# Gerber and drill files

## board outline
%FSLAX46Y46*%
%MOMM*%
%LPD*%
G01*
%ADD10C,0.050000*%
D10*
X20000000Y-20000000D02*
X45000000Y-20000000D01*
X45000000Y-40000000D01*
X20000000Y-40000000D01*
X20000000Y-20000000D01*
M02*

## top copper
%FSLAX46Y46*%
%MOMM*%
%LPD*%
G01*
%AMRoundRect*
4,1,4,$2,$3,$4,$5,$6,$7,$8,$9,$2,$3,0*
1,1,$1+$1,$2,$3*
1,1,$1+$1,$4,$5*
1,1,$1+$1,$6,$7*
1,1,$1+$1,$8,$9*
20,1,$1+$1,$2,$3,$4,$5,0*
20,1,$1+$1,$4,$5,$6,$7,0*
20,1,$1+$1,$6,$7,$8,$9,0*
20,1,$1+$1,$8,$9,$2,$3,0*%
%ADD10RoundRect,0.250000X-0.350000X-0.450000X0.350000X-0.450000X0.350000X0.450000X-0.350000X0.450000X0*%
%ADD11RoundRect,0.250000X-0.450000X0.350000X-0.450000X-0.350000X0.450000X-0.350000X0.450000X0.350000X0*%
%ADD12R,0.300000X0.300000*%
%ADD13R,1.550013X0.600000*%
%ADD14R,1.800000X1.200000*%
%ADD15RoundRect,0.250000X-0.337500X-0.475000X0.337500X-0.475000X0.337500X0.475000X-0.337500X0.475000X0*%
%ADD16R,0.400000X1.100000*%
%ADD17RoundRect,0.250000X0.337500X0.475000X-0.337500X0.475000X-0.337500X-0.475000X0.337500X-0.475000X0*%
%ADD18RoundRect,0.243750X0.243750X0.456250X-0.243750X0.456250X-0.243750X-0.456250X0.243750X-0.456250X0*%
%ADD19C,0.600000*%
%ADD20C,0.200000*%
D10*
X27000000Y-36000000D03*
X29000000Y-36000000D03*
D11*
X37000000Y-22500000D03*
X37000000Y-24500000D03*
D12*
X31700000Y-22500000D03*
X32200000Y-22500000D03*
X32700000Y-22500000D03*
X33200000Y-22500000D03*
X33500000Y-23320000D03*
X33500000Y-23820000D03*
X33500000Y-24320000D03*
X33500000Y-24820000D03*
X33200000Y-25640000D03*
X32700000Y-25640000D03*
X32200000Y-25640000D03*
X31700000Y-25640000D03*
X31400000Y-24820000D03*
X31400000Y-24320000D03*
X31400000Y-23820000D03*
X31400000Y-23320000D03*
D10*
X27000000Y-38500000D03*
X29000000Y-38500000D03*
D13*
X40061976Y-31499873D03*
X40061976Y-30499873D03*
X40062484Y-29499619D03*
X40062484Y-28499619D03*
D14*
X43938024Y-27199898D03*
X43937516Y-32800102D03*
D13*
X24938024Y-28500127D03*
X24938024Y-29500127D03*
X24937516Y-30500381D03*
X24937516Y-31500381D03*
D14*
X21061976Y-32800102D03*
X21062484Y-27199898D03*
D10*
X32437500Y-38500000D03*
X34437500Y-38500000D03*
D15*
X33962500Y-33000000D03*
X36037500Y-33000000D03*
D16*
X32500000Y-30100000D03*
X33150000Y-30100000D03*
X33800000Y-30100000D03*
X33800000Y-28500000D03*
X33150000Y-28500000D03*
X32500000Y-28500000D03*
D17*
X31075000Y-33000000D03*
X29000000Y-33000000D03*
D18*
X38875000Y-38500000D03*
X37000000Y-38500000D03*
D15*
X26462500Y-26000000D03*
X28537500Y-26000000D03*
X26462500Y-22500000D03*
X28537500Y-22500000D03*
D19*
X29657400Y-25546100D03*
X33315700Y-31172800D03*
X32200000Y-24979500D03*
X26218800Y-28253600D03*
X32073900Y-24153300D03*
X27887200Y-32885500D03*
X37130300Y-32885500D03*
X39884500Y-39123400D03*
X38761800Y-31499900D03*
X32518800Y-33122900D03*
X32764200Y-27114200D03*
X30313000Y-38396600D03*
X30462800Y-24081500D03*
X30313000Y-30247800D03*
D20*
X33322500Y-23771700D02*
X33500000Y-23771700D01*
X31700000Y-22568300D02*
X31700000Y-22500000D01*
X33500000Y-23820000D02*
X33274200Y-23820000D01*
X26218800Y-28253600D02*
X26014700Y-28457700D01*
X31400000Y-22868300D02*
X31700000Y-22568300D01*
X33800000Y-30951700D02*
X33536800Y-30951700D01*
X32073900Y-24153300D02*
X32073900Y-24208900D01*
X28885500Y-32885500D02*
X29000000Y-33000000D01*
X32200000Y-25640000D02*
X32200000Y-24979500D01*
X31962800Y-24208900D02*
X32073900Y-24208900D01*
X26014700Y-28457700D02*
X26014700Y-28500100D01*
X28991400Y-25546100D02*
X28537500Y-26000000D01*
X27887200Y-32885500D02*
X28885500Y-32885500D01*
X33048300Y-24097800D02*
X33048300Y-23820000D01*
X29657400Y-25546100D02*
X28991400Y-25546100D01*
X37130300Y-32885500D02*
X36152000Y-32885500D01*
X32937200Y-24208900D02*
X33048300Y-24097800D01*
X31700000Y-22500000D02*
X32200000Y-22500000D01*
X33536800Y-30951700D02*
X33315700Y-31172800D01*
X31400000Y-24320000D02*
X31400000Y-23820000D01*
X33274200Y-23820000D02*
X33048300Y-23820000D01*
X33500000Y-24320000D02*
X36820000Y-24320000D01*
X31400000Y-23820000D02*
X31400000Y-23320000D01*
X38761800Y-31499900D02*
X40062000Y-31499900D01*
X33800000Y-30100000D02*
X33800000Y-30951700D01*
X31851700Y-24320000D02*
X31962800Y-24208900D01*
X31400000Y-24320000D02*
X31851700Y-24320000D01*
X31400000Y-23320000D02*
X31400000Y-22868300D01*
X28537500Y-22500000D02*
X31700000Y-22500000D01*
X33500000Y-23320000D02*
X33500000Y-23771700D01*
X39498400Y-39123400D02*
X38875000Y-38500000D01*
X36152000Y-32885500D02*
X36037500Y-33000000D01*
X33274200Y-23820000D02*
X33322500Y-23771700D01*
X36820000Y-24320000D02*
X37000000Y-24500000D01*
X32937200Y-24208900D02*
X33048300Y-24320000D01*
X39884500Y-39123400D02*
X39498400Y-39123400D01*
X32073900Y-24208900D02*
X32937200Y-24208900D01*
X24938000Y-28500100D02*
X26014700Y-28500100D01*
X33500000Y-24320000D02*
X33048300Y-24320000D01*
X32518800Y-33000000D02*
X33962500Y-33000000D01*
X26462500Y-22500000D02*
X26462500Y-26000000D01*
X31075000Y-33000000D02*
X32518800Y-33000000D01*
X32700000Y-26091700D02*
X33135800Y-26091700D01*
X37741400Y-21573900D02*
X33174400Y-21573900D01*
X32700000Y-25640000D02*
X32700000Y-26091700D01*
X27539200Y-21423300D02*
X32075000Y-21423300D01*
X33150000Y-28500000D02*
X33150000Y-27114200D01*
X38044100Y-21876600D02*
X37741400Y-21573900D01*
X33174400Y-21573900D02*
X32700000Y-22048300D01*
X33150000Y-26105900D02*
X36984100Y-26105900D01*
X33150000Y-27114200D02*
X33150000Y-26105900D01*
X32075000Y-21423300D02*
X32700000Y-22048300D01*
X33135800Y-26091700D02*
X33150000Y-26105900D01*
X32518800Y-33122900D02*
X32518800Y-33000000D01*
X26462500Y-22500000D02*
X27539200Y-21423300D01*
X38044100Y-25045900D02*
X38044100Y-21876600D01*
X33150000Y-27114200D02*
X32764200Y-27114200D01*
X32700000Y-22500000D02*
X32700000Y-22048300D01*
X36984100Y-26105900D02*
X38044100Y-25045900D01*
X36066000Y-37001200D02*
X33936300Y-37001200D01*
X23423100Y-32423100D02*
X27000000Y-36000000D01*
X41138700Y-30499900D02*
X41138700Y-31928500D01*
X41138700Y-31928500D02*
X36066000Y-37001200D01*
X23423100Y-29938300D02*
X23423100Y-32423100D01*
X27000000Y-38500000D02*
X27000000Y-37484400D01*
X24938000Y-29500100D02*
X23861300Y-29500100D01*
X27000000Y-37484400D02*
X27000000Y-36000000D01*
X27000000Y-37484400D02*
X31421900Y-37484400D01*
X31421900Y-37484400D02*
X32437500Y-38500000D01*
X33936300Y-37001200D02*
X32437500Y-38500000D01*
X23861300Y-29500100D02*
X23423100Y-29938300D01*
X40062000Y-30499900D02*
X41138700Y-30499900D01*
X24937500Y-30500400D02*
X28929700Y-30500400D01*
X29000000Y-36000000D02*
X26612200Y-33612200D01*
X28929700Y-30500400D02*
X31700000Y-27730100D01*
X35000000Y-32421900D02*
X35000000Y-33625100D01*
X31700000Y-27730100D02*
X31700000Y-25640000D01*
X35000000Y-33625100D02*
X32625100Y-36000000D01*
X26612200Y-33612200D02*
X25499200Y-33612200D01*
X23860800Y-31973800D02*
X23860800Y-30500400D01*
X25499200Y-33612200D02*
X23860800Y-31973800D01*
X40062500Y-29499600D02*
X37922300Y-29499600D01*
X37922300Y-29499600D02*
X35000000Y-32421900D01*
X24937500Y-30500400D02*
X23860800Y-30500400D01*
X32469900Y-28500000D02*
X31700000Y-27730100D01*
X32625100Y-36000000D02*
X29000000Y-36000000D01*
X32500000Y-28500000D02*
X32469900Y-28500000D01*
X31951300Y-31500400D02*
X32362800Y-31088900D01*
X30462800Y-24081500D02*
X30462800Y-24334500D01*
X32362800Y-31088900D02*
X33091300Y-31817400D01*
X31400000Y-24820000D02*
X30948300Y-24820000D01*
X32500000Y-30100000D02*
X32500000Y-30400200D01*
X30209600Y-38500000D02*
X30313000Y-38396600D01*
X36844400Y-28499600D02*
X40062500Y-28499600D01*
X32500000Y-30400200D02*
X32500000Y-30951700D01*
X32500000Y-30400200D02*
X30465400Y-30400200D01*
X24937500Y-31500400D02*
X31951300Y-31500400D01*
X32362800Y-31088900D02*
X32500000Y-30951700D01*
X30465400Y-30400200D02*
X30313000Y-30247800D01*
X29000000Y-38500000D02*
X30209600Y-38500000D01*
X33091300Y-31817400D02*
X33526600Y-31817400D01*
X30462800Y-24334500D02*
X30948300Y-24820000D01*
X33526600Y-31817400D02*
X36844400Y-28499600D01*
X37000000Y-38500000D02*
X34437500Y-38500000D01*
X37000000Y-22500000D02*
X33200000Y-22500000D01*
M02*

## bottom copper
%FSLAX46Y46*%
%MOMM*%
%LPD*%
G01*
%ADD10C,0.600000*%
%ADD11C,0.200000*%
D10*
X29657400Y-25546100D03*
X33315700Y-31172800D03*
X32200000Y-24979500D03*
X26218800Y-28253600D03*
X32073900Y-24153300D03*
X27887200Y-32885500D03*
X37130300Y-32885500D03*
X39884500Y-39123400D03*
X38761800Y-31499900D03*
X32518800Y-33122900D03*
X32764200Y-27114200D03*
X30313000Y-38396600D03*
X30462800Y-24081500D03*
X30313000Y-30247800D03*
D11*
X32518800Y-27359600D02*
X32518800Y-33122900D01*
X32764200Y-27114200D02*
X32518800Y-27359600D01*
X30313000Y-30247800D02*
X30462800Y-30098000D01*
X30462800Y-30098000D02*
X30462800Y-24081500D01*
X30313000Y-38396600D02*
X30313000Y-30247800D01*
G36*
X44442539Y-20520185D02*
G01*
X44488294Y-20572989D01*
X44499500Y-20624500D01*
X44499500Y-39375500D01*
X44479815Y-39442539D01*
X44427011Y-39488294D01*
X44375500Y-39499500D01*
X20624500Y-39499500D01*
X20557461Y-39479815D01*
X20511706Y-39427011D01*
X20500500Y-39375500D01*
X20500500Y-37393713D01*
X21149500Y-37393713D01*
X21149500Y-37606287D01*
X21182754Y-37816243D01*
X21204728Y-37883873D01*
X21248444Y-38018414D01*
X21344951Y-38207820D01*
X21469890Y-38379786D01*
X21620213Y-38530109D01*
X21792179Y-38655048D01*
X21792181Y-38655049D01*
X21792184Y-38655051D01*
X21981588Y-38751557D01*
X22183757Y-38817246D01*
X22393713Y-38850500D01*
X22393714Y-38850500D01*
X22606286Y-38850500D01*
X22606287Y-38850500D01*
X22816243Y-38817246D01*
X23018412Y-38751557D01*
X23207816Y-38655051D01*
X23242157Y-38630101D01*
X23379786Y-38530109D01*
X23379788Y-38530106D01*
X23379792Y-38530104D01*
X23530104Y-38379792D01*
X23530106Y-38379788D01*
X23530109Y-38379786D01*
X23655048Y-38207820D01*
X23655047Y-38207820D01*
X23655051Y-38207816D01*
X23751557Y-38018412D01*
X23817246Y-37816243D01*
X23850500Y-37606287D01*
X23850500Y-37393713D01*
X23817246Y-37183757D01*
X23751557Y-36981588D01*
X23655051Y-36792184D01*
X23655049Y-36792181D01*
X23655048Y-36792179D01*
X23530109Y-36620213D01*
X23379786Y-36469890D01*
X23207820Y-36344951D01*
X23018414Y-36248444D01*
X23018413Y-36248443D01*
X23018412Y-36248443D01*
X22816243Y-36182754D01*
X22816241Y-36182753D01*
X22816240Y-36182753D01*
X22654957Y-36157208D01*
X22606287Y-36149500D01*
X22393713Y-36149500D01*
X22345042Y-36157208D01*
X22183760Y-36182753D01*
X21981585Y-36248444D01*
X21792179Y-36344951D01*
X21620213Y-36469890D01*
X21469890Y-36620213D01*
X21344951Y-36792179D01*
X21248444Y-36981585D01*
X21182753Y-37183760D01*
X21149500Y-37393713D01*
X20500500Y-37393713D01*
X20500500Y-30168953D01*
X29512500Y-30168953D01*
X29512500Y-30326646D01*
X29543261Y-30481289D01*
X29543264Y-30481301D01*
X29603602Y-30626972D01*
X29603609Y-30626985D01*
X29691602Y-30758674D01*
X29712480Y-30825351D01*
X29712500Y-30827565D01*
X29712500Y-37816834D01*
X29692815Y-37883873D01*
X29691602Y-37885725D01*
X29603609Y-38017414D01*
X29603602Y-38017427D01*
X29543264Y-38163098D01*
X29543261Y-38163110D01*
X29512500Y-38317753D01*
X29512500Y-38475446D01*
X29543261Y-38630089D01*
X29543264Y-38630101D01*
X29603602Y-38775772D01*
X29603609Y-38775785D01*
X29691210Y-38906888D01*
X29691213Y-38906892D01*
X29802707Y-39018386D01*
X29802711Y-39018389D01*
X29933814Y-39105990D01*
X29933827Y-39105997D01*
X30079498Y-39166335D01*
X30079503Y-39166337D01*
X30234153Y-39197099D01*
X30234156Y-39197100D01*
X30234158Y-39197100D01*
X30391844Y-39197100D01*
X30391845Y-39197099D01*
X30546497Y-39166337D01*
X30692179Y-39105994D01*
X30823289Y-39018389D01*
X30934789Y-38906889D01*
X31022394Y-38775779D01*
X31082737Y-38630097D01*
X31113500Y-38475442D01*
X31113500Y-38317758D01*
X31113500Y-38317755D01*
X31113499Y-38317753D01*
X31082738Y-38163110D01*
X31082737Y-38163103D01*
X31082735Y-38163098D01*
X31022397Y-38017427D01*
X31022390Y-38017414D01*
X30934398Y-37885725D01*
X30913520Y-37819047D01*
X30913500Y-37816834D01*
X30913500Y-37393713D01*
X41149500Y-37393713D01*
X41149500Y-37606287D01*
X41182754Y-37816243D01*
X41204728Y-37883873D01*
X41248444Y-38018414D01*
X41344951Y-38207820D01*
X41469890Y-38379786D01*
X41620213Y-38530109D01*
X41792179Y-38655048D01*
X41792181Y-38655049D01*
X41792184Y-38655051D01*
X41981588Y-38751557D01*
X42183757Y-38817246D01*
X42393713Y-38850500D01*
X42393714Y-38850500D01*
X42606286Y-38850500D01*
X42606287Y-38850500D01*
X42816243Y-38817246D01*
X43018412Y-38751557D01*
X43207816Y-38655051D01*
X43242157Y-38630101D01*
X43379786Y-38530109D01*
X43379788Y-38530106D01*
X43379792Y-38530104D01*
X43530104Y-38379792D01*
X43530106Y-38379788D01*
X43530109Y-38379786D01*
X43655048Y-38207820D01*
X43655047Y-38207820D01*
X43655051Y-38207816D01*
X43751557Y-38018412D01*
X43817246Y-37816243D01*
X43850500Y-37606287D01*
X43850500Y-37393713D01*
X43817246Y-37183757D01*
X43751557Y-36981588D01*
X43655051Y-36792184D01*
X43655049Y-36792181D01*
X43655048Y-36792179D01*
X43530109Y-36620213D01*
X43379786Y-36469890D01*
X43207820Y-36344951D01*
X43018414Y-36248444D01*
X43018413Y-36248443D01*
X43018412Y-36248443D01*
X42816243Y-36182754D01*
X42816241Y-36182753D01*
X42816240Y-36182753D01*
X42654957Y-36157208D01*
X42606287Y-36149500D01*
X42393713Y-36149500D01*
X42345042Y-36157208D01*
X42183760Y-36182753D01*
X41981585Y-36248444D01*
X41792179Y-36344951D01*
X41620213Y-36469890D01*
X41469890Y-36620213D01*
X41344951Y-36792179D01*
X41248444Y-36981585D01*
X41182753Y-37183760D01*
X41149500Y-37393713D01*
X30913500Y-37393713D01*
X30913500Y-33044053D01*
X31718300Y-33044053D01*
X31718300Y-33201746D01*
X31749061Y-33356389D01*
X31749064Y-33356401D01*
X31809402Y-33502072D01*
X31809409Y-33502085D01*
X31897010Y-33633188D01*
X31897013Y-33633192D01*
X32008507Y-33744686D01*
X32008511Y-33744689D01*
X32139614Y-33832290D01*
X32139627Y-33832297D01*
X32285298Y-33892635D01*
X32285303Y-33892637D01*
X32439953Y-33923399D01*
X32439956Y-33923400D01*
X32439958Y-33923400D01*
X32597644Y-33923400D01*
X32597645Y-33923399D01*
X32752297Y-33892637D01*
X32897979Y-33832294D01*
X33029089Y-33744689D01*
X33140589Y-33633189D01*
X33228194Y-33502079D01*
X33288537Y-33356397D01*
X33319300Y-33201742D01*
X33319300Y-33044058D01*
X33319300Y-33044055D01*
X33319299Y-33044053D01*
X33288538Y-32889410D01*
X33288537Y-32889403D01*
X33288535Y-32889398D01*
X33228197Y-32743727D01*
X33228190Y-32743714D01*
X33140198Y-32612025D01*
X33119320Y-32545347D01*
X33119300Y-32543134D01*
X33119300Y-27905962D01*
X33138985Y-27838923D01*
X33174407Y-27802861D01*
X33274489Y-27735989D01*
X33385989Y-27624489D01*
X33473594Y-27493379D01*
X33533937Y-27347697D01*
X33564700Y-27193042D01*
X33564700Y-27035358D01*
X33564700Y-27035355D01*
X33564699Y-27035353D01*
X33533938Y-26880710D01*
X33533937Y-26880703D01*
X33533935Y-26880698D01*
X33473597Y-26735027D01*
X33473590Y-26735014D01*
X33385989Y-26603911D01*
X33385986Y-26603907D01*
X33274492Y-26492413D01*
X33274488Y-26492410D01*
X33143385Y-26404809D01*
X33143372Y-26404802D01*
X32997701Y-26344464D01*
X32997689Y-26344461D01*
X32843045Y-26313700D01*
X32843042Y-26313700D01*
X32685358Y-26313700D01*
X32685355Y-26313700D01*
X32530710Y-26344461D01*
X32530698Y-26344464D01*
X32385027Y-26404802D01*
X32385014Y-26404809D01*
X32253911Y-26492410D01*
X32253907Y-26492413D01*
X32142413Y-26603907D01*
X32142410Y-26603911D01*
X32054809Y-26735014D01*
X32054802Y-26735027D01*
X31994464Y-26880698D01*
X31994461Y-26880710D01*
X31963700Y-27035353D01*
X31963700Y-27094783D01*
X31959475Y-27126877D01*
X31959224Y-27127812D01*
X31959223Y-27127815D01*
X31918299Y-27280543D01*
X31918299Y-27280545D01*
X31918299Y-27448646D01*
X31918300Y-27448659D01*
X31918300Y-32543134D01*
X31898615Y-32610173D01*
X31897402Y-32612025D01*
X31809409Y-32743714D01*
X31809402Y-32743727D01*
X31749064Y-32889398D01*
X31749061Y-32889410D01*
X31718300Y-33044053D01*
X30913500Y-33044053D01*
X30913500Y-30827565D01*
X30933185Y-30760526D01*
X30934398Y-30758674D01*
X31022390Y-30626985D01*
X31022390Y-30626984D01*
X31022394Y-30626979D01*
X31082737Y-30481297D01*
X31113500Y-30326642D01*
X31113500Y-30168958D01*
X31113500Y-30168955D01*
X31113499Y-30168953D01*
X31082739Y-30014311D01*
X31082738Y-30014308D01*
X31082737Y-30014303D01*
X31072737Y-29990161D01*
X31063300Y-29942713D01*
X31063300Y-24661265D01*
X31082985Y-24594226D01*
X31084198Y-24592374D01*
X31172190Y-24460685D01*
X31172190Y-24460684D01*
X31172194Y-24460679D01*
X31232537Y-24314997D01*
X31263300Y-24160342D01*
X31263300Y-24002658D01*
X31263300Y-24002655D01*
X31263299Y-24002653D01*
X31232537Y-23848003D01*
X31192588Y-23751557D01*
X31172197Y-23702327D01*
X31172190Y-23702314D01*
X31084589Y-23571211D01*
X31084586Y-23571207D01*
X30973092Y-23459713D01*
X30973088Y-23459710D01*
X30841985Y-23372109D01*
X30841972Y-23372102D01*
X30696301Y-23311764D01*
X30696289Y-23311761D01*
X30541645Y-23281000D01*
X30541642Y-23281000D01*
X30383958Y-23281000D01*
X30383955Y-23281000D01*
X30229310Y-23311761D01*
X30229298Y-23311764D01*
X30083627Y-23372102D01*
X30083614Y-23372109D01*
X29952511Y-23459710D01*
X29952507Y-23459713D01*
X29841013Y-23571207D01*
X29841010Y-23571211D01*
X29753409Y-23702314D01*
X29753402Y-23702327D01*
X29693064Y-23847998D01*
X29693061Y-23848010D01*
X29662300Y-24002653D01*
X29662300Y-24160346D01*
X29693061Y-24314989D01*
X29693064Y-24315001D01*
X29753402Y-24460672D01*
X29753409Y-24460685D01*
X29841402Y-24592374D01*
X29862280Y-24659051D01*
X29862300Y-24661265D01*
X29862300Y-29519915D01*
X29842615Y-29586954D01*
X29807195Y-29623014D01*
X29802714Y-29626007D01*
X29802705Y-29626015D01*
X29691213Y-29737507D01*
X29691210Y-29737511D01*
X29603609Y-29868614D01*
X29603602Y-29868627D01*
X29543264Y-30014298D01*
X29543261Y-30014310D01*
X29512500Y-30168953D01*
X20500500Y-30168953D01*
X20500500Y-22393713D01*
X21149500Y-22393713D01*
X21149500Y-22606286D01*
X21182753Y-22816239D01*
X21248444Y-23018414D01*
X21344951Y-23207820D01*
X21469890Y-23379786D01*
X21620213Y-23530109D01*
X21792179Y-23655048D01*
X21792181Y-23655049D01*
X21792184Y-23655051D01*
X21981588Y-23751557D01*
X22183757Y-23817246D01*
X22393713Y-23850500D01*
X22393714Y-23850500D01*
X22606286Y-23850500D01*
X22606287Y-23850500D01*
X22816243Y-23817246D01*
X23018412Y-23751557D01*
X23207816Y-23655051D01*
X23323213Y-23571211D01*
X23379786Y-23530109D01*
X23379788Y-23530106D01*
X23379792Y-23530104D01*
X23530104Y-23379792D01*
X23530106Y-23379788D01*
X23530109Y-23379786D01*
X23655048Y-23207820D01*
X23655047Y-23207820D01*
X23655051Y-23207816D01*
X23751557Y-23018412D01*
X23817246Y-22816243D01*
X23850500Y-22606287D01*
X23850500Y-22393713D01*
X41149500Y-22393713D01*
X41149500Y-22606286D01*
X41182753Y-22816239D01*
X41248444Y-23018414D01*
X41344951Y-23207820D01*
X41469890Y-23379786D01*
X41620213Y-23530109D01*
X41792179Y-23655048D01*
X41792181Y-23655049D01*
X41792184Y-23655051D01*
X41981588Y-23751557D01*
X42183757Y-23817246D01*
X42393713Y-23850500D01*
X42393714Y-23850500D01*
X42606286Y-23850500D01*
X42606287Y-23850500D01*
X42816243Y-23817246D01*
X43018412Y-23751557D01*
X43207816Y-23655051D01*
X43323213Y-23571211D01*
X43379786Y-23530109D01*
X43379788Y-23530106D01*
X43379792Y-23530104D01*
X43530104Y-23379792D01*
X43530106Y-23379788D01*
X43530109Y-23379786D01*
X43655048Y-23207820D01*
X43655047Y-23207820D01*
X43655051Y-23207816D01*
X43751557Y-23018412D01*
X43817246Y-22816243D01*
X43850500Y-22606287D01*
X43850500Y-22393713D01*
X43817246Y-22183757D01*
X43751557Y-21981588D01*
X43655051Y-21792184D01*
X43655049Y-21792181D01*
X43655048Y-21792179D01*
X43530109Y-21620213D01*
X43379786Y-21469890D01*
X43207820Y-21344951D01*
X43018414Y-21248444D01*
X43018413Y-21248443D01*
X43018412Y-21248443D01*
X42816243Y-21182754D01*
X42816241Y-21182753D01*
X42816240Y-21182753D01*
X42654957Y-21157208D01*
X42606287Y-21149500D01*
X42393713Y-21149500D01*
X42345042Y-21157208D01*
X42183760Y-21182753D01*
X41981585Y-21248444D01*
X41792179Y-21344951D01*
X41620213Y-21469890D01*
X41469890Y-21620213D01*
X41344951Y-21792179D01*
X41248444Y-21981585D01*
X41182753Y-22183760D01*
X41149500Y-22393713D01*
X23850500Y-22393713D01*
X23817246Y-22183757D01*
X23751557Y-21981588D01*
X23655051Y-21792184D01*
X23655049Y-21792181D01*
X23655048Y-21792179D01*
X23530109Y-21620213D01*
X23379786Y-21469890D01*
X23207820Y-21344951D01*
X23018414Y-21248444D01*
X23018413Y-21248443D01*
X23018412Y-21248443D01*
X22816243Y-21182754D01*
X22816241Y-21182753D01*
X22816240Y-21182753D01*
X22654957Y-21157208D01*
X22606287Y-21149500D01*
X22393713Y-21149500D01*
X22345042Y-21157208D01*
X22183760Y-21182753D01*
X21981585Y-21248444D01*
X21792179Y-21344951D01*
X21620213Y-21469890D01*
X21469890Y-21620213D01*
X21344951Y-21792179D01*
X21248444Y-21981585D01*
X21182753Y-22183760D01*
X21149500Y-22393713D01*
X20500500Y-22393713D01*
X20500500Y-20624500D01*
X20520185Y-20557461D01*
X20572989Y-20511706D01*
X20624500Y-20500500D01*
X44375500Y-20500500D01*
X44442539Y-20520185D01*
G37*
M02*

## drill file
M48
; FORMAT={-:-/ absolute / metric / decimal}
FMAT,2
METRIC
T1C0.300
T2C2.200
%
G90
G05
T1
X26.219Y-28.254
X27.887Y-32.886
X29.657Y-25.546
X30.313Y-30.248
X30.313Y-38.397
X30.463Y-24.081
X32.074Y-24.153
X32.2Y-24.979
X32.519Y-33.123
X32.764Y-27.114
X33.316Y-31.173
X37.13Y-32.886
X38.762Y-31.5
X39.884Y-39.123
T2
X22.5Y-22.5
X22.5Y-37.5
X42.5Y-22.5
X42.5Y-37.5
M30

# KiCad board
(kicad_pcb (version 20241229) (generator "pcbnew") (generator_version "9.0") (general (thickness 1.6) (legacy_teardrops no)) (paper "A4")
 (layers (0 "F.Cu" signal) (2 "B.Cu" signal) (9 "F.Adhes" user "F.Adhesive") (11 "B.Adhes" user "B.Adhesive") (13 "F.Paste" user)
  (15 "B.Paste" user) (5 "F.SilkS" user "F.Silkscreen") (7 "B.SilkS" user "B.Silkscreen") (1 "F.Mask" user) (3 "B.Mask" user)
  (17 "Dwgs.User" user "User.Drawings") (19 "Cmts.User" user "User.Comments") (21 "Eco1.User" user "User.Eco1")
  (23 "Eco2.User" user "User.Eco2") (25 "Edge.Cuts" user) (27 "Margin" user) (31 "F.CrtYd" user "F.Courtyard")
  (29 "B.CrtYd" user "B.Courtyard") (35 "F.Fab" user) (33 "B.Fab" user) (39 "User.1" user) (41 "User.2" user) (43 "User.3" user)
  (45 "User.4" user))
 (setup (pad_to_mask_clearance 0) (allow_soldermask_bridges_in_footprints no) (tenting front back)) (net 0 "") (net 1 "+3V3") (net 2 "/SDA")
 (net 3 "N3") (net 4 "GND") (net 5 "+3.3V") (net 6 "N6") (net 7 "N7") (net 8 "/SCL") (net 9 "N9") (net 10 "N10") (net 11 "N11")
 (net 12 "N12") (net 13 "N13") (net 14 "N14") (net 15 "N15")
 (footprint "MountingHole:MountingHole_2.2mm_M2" (layer "F.Cu") (at 22.5 22.5)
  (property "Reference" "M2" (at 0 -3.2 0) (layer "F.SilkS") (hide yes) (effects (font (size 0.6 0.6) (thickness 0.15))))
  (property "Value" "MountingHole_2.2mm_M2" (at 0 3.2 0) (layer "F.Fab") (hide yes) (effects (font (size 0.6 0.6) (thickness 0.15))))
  (pad "" np_thru_hole circle (at 0 0) (size 2.2 2.2) (drill 2.2) (layers "*.Cu" "*.Mask")))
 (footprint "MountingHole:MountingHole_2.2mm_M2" (layer "F.Cu") (at 42.5 22.5)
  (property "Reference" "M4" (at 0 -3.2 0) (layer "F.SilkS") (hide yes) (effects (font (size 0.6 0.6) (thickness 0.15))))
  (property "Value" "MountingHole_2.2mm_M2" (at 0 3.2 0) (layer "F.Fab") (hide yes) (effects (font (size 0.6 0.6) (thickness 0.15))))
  (pad "" np_thru_hole circle (at 0 0) (size 2.2 2.2) (drill 2.2) (layers "*.Cu" "*.Mask")))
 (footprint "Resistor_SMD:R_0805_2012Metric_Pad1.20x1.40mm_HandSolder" (layer "F.Cu") (at 28 36)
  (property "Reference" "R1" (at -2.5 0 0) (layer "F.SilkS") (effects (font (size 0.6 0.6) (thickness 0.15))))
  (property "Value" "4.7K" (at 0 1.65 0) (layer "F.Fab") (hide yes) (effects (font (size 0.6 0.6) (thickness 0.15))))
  (pad "1" smd roundrect (at -1 0) (size 1.2 1.4) (layers "F.Cu" "F.Mask" "F.Paste") (roundrect_rratio 0.208333) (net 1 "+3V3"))
  (pad "2" smd roundrect (at 1 0) (size 1.2 1.4) (layers "F.Cu" "F.Mask" "F.Paste") (roundrect_rratio 0.208333) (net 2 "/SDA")))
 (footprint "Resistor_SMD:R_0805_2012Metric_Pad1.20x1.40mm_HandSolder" (layer "F.Cu") (at 37 23.5 -90)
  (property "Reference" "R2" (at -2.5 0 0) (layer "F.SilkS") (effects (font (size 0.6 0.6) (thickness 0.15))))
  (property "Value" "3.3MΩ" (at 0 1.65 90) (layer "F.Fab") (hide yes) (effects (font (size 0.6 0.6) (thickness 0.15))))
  (pad "1" smd roundrect (at -1 0 270) (size 1.2 1.4) (layers "F.Cu" "F.Mask" "F.Paste") (roundrect_rratio 0.208333) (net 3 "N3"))
  (pad "2" smd roundrect (at 1 0 270) (size 1.2 1.4) (layers "F.Cu" "F.Mask" "F.Paste") (roundrect_rratio 0.208333) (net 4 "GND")))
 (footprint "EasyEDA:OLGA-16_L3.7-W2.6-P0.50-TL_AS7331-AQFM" (layer "F.Cu") (at 32.45 24.07)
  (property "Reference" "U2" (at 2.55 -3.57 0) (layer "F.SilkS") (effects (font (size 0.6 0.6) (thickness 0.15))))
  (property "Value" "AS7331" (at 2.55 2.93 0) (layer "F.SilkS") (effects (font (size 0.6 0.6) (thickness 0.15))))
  (pad "1" smd rect (at -0.75 -1.57) (size 0.3 0.3) (layers "F.Cu" "F.Mask" "F.Paste") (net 4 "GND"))
  (pad "2" smd rect (at -0.25 -1.57) (size 0.3 0.3) (layers "F.Cu" "F.Mask" "F.Paste") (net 4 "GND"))
  (pad "3" smd rect (at 0.25 -1.57) (size 0.3 0.3) (layers "F.Cu" "F.Mask" "F.Paste") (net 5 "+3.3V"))
  (pad "4" smd rect (at 0.75 -1.57) (size 0.3 0.3) (layers "F.Cu" "F.Mask" "F.Paste") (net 3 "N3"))
  (pad "5" smd rect (at 1.05 -0.75) (size 0.3 0.3) (layers "F.Cu" "F.Mask" "F.Paste") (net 4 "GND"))
  (pad "6" smd rect (at 1.05 -0.25) (size 0.3 0.3) (layers "F.Cu" "F.Mask" "F.Paste") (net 4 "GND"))
  (pad "7" smd rect (at 1.05 0.25) (size 0.3 0.3) (layers "F.Cu" "F.Mask" "F.Paste") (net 4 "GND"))
  (pad "8" smd rect (at 1.05 0.75) (size 0.3 0.3) (layers "F.Cu" "F.Mask" "F.Paste") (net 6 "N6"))
  (pad "9" smd rect (at 0.75 1.57) (size 0.3 0.3) (layers "F.Cu" "F.Mask" "F.Paste") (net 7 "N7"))
  (pad "10" smd rect (at 0.25 1.57) (size 0.3 0.3) (layers "F.Cu" "F.Mask" "F.Paste") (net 5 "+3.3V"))
  (pad "11" smd rect (at -0.25 1.57) (size 0.3 0.3) (layers "F.Cu" "F.Mask" "F.Paste") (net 4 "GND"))
  (pad "12" smd rect (at -0.75 1.57) (size 0.3 0.3) (layers "F.Cu" "F.Mask" "F.Paste") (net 2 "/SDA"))
  (pad "13" smd rect (at -1.05 0.75) (size 0.3 0.3) (layers "F.Cu" "F.Mask" "F.Paste") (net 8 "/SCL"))
  (pad "14" smd rect (at -1.05 0.25) (size 0.3 0.3) (layers "F.Cu" "F.Mask" "F.Paste") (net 4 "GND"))
  (pad "15" smd rect (at -1.05 -0.25) (size 0.3 0.3) (layers "F.Cu" "F.Mask" "F.Paste") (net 4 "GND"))
  (pad "16" smd rect (at -1.05 -0.75) (size 0.3 0.3) (layers "F.Cu" "F.Mask" "F.Paste") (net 4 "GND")))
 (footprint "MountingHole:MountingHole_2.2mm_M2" (layer "F.Cu") (at 42.5 37.5)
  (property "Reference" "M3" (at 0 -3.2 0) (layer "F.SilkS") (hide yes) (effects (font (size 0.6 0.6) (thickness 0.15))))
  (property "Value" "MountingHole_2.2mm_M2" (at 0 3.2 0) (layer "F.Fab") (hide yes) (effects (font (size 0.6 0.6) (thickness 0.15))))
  (pad "" np_thru_hole circle (at 0 0) (size 2.2 2.2) (drill 2.2) (layers "*.Cu" "*.Mask")))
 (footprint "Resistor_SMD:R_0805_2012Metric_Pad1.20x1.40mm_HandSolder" (layer "F.Cu") (at 28 38.5)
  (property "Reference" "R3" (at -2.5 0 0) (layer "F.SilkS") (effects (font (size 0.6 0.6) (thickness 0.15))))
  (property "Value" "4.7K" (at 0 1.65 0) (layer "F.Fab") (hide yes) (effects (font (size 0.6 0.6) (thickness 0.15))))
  (pad "1" smd roundrect (at -1 0) (size 1.2 1.4) (layers "F.Cu" "F.Mask" "F.Paste") (roundrect_rratio 0.208333) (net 1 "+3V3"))
  (pad "2" smd roundrect (at 1 0) (size 1.2 1.4) (layers "F.Cu" "F.Mask" "F.Paste") (roundrect_rratio 0.208333) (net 8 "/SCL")))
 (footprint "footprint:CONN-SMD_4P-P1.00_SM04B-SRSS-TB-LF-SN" (layer "F.Cu") (at 42 30 90)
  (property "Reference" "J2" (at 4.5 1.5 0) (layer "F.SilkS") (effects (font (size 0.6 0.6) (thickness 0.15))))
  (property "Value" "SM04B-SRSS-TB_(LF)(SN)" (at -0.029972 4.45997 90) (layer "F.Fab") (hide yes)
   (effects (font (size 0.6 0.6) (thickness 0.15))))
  (pad "1" smd rect (at -1.499873 -1.938024 90) (size 0.6 1.550013) (layers "F.Cu" "F.Mask" "F.Paste") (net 4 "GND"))
  (pad "2" smd rect (at -0.499873 -1.938024 90) (size 0.6 1.550013) (layers "F.Cu" "F.Mask" "F.Paste") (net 1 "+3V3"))
  (pad "3" smd rect (at 0.500381 -1.937516 90) (size 0.6 1.550013) (layers "F.Cu" "F.Mask" "F.Paste") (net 2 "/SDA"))
  (pad "4" smd rect (at 1.500381 -1.937516 90) (size 0.6 1.550013) (layers "F.Cu" "F.Mask" "F.Paste") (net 8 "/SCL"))
  (pad "5" smd rect (at 2.800102 1.938024 90) (size 1.2 1.8) (layers "F.Cu" "F.Mask" "F.Paste") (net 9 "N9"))
  (pad "6" smd rect (at -2.800102 1.937516 90) (size 1.2 1.8) (layers "F.Cu" "F.Mask" "F.Paste") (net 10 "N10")))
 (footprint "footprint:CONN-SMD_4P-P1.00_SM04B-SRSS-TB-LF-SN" (layer "F.Cu") (at 23 30 -90)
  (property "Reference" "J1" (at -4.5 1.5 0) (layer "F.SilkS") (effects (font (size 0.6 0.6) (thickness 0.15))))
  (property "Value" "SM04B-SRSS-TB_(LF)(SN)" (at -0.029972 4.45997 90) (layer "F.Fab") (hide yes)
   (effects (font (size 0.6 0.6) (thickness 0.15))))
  (pad "1" smd rect (at -1.499873 -1.938024 270) (size 0.6 1.550013) (layers "F.Cu" "F.Mask" "F.Paste") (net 4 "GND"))
  (pad "2" smd rect (at -0.499873 -1.938024 270) (size 0.6 1.550013) (layers "F.Cu" "F.Mask" "F.Paste") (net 1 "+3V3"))
  (pad "3" smd rect (at 0.500381 -1.937516 270) (size 0.6 1.550013) (layers "F.Cu" "F.Mask" "F.Paste") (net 2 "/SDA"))
  (pad "4" smd rect (at 1.500381 -1.937516 270) (size 0.6 1.550013) (layers "F.Cu" "F.Mask" "F.Paste") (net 8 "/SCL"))
  (pad "5" smd rect (at 2.800102 1.938024 270) (size 1.2 1.8) (layers "F.Cu" "F.Mask" "F.Paste") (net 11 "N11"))
  (pad "6" smd rect (at -2.800102 1.937516 270) (size 1.2 1.8) (layers "F.Cu" "F.Mask" "F.Paste") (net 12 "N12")))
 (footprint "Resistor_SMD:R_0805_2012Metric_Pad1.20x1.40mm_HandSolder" (layer "F.Cu") (at 33.4375 38.5)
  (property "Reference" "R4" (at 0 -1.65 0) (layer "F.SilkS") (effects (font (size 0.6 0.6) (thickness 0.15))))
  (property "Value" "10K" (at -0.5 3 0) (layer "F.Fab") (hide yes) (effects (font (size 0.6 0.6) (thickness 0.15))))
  (pad "1" smd roundrect (at -1 0) (size 1.2 1.4) (layers "F.Cu" "F.Mask" "F.Paste") (roundrect_rratio 0.208333) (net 1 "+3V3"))
  (pad "2" smd roundrect (at 1 0) (size 1.2 1.4) (layers "F.Cu" "F.Mask" "F.Paste") (roundrect_rratio 0.208333) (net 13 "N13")))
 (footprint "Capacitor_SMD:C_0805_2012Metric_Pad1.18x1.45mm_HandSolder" (layer "F.Cu") (at 35 33)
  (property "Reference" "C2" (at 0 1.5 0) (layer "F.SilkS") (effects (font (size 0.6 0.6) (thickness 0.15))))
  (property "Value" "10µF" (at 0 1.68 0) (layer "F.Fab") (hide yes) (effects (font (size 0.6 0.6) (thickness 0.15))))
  (pad "1" smd roundrect (at -1.0375 0) (size 1.175 1.45) (layers "F.Cu" "F.Mask" "F.Paste") (roundrect_rratio 0.212766) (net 5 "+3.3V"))
  (pad "2" smd roundrect (at 1.0375 0) (size 1.175 1.45) (layers "F.Cu" "F.Mask" "F.Paste") (roundrect_rratio 0.212766) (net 4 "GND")))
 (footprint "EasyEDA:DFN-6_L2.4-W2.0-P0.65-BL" (layer "F.Cu") (at 33.15 29.3)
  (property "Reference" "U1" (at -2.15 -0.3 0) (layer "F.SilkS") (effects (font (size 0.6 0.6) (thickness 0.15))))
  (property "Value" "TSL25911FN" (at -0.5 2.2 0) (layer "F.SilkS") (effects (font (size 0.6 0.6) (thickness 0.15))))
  (pad "1" smd rect (at -0.65 0.8) (size 0.4 1.1) (layers "F.Cu" "F.Mask" "F.Paste") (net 8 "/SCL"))
  (pad "2" smd rect (at 0 0.8) (size 0.4 1.1) (layers "F.Cu" "F.Mask" "F.Paste") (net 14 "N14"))
  (pad "3" smd rect (at 0.65 0.8) (size 0.4 1.1) (layers "F.Cu" "F.Mask" "F.Paste") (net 4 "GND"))
  (pad "4" smd rect (at 0.65 -0.8) (size 0.4 1.1) (layers "F.Cu" "F.Mask" "F.Paste") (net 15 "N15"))
  (pad "5" smd rect (at 0 -0.8) (size 0.4 1.1) (layers "F.Cu" "F.Mask" "F.Paste") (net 5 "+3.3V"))
  (pad "6" smd rect (at -0.65 -0.8) (size 0.4 1.1) (layers "F.Cu" "F.Mask" "F.Paste") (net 2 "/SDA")))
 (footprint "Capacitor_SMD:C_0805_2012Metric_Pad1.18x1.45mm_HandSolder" (layer "F.Cu") (at 30.0375 33 180)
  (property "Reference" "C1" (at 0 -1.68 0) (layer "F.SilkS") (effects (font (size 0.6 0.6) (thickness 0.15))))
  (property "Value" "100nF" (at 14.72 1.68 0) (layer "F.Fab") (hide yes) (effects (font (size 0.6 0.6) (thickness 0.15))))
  (pad "1" smd roundrect (at -1.0375 0 180) (size 1.175 1.45) (layers "F.Cu" "F.Mask" "F.Paste") (roundrect_rratio 0.212766) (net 5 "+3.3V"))
  (pad "2" smd roundrect (at 1.0375 0 180) (size 1.175 1.45) (layers "F.Cu" "F.Mask" "F.Paste") (roundrect_rratio 0.212766) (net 4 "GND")))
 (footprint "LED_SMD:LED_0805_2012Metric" (layer "F.Cu") (at 37.9375 38.5 180)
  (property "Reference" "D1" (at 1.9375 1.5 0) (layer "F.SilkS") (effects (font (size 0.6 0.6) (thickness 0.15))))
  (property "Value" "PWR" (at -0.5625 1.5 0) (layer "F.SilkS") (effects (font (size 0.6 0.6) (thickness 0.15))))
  (pad "1" smd roundrect (at -0.9375 0 180) (size 0.975 1.4) (layers "F.Cu" "F.Mask" "F.Paste") (roundrect_rratio 0.25) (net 4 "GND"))
  (pad "2" smd roundrect (at 0.9375 0 180) (size 0.975 1.4) (layers "F.Cu" "F.Mask" "F.Paste") (roundrect_rratio 0.25) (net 13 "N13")))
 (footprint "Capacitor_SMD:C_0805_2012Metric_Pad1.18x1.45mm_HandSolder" (layer "F.Cu") (at 27.5 26)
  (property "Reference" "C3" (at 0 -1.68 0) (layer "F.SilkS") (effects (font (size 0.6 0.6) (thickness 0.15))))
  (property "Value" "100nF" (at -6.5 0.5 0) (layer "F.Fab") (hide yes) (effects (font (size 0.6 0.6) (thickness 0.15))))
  (pad "1" smd roundrect (at -1.0375 0) (size 1.175 1.45) (layers "F.Cu" "F.Mask" "F.Paste") (roundrect_rratio 0.212766) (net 5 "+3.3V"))
  (pad "2" smd roundrect (at 1.0375 0) (size 1.175 1.45) (layers "F.Cu" "F.Mask" "F.Paste") (roundrect_rratio 0.212766) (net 4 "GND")))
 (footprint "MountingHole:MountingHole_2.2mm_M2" (layer "F.Cu") (at 22.5 37.5)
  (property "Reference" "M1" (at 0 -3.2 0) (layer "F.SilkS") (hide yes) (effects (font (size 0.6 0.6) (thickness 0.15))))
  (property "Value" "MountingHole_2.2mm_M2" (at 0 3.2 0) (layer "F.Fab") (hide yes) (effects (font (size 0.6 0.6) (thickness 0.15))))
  (pad "" np_thru_hole circle (at 0 0) (size 2.2 2.2) (drill 2.2) (layers "*.Cu" "*.Mask")))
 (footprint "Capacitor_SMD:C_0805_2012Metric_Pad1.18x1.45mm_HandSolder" (layer "F.Cu") (at 27.5 22.5)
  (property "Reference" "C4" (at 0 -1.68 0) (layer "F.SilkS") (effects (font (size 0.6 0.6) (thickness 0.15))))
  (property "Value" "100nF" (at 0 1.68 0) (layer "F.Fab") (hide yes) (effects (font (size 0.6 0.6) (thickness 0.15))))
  (pad "1" smd roundrect (at -1.0375 0) (size 1.175 1.45) (layers "F.Cu" "F.Mask" "F.Paste") (roundrect_rratio 0.212766) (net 5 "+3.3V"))
  (pad "2" smd roundrect (at 1.0375 0) (size 1.175 1.45) (layers "F.Cu" "F.Mask" "F.Paste") (roundrect_rratio 0.212766) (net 4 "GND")))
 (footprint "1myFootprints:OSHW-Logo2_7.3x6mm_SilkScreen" (layer "B.Cu") (at 37.5 23.5 180)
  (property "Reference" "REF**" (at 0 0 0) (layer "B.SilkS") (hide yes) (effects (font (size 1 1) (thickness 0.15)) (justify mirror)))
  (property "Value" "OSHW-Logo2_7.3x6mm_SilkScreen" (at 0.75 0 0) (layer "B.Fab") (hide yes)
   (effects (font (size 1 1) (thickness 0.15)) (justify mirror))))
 (gr_rect (start 20 20) (end 45 40) (stroke (width 0.05) (type solid)) (fill no) (layer "Edge.Cuts"))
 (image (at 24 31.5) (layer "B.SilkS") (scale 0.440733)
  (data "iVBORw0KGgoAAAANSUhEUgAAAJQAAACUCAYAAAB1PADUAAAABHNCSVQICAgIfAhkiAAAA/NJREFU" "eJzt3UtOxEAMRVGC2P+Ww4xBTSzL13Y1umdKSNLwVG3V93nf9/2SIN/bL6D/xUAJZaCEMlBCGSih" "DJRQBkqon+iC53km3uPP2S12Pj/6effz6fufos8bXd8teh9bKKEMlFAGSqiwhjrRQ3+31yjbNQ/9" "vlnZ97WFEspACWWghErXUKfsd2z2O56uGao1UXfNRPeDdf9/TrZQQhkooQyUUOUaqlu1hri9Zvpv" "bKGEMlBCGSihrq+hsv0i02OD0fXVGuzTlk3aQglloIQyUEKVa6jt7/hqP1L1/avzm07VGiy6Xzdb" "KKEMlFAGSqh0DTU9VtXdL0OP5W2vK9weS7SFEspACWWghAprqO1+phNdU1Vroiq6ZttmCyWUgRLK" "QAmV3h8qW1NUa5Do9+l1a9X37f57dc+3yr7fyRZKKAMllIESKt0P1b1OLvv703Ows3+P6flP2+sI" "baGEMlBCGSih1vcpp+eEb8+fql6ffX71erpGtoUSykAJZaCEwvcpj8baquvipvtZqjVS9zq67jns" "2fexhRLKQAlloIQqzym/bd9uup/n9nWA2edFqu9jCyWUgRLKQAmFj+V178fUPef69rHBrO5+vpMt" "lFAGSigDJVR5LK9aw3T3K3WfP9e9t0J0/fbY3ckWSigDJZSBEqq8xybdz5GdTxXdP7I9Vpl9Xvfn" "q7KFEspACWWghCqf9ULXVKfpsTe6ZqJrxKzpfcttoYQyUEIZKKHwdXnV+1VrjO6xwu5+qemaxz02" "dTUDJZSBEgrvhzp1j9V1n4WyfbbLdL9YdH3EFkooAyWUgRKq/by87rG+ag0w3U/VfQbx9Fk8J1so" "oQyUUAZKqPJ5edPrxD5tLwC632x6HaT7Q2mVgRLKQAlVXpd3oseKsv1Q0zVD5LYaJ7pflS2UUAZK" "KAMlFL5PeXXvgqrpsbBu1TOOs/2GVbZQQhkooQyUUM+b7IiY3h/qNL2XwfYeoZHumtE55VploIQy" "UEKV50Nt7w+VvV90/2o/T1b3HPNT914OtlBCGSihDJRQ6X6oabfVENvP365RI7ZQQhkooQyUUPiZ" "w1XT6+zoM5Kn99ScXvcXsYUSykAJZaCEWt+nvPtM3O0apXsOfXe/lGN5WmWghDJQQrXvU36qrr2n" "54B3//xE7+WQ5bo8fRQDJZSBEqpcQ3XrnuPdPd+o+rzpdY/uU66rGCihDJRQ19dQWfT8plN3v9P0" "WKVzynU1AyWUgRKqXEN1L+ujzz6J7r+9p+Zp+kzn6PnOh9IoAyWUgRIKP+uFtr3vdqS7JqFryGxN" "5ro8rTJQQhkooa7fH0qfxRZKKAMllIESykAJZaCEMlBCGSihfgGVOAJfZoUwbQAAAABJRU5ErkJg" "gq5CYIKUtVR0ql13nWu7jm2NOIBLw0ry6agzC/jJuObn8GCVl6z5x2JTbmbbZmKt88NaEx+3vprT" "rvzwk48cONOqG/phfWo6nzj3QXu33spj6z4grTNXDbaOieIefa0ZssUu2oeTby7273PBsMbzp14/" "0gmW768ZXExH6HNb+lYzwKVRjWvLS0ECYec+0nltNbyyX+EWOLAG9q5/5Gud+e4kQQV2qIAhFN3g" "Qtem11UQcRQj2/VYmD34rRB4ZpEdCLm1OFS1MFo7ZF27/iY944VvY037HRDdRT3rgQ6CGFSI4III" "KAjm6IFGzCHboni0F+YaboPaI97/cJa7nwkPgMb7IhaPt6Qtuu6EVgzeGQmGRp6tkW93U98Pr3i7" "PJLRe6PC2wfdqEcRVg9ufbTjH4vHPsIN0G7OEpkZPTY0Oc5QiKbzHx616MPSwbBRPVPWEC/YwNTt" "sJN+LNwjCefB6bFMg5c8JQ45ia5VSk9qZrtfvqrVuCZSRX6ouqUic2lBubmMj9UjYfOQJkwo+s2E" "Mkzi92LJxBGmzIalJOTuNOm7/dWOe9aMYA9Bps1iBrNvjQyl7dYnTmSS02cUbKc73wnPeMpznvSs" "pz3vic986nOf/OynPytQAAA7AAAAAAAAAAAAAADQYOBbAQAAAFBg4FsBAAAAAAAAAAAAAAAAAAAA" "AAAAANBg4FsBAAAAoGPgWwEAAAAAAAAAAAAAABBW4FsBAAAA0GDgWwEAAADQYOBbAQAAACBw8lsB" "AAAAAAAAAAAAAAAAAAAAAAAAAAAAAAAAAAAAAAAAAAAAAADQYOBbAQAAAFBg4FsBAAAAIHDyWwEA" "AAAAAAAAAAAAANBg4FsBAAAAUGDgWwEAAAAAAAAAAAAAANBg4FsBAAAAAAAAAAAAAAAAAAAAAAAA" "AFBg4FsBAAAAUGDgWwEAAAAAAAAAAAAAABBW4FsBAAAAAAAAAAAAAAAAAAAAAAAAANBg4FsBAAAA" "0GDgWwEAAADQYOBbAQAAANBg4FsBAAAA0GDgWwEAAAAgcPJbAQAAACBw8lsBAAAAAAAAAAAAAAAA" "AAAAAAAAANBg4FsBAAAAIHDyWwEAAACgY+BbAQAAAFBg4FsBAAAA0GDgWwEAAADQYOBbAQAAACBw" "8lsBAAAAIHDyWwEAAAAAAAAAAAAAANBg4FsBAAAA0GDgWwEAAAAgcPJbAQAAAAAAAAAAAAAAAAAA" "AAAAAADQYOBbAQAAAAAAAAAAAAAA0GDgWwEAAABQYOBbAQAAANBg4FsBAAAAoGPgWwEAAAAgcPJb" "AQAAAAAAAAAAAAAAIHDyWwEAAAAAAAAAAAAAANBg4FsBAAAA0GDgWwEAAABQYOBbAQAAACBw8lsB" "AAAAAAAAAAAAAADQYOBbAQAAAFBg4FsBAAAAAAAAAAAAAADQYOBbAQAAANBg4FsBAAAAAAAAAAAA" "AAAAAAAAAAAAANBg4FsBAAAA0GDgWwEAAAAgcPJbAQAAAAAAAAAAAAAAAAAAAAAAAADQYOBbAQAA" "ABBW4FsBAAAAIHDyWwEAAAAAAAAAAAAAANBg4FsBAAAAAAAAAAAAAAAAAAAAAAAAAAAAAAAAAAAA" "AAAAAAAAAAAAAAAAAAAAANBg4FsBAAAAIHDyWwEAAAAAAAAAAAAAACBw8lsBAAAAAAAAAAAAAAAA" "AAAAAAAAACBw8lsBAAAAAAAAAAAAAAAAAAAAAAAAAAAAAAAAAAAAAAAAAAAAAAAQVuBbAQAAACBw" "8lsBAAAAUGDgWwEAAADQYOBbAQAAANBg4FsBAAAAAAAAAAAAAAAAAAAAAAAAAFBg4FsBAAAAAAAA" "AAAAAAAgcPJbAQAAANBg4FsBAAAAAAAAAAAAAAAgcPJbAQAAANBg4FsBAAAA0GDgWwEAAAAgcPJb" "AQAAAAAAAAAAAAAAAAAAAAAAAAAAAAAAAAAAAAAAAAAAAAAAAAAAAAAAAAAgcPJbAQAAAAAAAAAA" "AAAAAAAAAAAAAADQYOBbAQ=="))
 (segment (start 33.3225 23.7717) (end 33.5 23.7717) (width 0.2) (layer "F.Cu") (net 4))
 (segment (start 31.7 22.5683) (end 31.7 22.5) (width 0.2) (layer "F.Cu") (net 4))
 (segment (start 33.5 23.82) (end 33.2742 23.82) (width 0.2) (layer "F.Cu") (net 4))
 (segment (start 26.2188 28.2536) (end 26.0147 28.4577) (width 0.2) (layer "F.Cu") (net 4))
 (segment (start 31.4 22.8683) (end 31.7 22.5683) (width 0.2) (layer "F.Cu") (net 4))
 (segment (start 33.8 30.9517) (end 33.5368 30.9517) (width 0.2) (layer "F.Cu") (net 4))
 (segment (start 32.0739 24.1533) (end 32.0739 24.2089) (width 0.2) (layer "F.Cu") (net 4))
 (segment (start 28.8855 32.8855) (end 29 33) (width 0.2) (layer "F.Cu") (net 4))
 (segment (start 32.2 25.64) (end 32.2 24.9795) (width 0.2) (layer "F.Cu") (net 4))
 (segment (start 31.9628 24.2089) (end 32.0739 24.2089) (width 0.2) (layer "F.Cu") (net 4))
 (segment (start 26.0147 28.4577) (end 26.0147 28.5001) (width 0.2) (layer "F.Cu") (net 4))
 (segment (start 28.9914 25.5461) (end 28.5375 26) (width 0.2) (layer "F.Cu") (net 4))
 (segment (start 27.8872 32.8855) (end 28.8855 32.8855) (width 0.2) (layer "F.Cu") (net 4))
 (segment (start 33.0483 24.0978) (end 33.0483 23.82) (width 0.2) (layer "F.Cu") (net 4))
 (segment (start 29.6574 25.5461) (end 28.9914 25.5461) (width 0.2) (layer "F.Cu") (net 4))
 (segment (start 37.1303 32.8855) (end 36.152 32.8855) (width 0.2) (layer "F.Cu") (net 4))
 (segment (start 32.9372 24.2089) (end 33.0483 24.0978) (width 0.2) (layer "F.Cu") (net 4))
 (segment (start 31.7 22.5) (end 32.2 22.5) (width 0.2) (layer "F.Cu") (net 4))
 (segment (start 33.5368 30.9517) (end 33.3157 31.1728) (width 0.2) (layer "F.Cu") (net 4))
 (segment (start 31.4 24.32) (end 31.4 23.82) (width 0.2) (layer "F.Cu") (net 4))
 (segment (start 33.2742 23.82) (end 33.0483 23.82) (width 0.2) (layer "F.Cu") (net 4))
 (segment (start 33.5 24.32) (end 36.82 24.32) (width 0.2) (layer "F.Cu") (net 4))
 (segment (start 31.4 23.82) (end 31.4 23.32) (width 0.2) (layer "F.Cu") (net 4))
 (segment (start 38.7618 31.4999) (end 40.062 31.4999) (width 0.2) (layer "F.Cu") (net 4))
 (segment (start 33.8 30.1) (end 33.8 30.9517) (width 0.2) (layer "F.Cu") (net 4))
 (segment (start 31.8517 24.32) (end 31.9628 24.2089) (width 0.2) (layer "F.Cu") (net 4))
 (segment (start 31.4 24.32) (end 31.8517 24.32) (width 0.2) (layer "F.Cu") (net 4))
 (segment (start 31.4 23.32) (end 31.4 22.8683) (width 0.2) (layer "F.Cu") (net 4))
 (segment (start 28.5375 22.5) (end 31.7 22.5) (width 0.2) (layer "F.Cu") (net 4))
 (segment (start 33.5 23.32) (end 33.5 23.7717) (width 0.2) (layer "F.Cu") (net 4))
 (segment (start 39.4984 39.1234) (end 38.875 38.5) (width 0.2) (layer "F.Cu") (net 4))
 (segment (start 36.152 32.8855) (end 36.0375 33) (width 0.2) (layer "F.Cu") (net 4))
 (segment (start 33.2742 23.82) (end 33.3225 23.7717) (width 0.2) (layer "F.Cu") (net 4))
 (segment (start 36.82 24.32) (end 37 24.5) (width 0.2) (layer "F.Cu") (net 4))
 (segment (start 32.9372 24.2089) (end 33.0483 24.32) (width 0.2) (layer "F.Cu") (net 4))
 (segment (start 39.8845 39.1234) (end 39.4984 39.1234) (width 0.2) (layer "F.Cu") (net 4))
 (segment (start 32.0739 24.2089) (end 32.9372 24.2089) (width 0.2) (layer "F.Cu") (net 4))
 (segment (start 24.938 28.5001) (end 26.0147 28.5001) (width 0.2) (layer "F.Cu") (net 4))
 (segment (start 33.5 24.32) (end 33.0483 24.32) (width 0.2) (layer "F.Cu") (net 4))
 (via (at 29.6574 25.5461) (size 0.6) (drill 0.3) (layers "F.Cu" "B.Cu") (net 4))
 (via (at 33.3157 31.1728) (size 0.6) (drill 0.3) (layers "F.Cu" "B.Cu") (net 4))
 (via (at 32.2 24.9795) (size 0.6) (drill 0.3) (layers "F.Cu" "B.Cu") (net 4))
 (via (at 26.2188 28.2536) (size 0.6) (drill 0.3) (layers "F.Cu" "B.Cu") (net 4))
 (via (at 32.0739 24.1533) (size 0.6) (drill 0.3) (layers "F.Cu" "B.Cu") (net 4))
 (via (at 27.8872 32.8855) (size 0.6) (drill 0.3) (layers "F.Cu" "B.Cu") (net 4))
 (via (at 37.1303 32.8855) (size 0.6) (drill 0.3) (layers "F.Cu" "B.Cu") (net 4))
 (via (at 39.8845 39.1234) (size 0.6) (drill 0.3) (layers "F.Cu" "B.Cu") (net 4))
 (via (at 38.7618 31.4999) (size 0.6) (drill 0.3) (layers "F.Cu" "B.Cu") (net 4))
 (segment (start 32.5188 33) (end 33.9625 33) (width 0.2) (layer "F.Cu") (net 5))
 (segment (start 26.4625 22.5) (end 26.4625 26) (width 0.2) (layer "F.Cu") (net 5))
 (segment (start 31.075 33) (end 32.5188 33) (width 0.2) (layer "F.Cu") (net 5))
 (segment (start 32.7 26.0917) (end 33.1358 26.0917) (width 0.2) (layer "F.Cu") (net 5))
 (segment (start 37.7414 21.5739) (end 33.1744 21.5739) (width 0.2) (layer "F.Cu") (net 5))
 (segment (start 32.7 25.64) (end 32.7 26.0917) (width 0.2) (layer "F.Cu") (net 5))
 (segment (start 27.5392 21.4233) (end 32.075 21.4233) (width 0.2) (layer "F.Cu") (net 5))
 (segment (start 33.15 28.5) (end 33.15 27.1142) (width 0.2) (layer "F.Cu") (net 5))
 (segment (start 38.0441 21.8766) (end 37.7414 21.5739) (width 0.2) (layer "F.Cu") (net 5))
 (segment (start 33.1744 21.5739) (end 32.7 22.0483) (width 0.2) (layer "F.Cu") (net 5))
 (segment (start 33.15 26.1059) (end 36.9841 26.1059) (width 0.2) (layer "F.Cu") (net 5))
 (segment (start 33.15 27.1142) (end 33.15 26.1059) (width 0.2) (layer "F.Cu") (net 5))
 (segment (start 32.075 21.4233) (end 32.7 22.0483) (width 0.2) (layer "F.Cu") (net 5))
 (segment (start 33.1358 26.0917) (end 33.15 26.1059) (width 0.2) (layer "F.Cu") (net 5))
 (segment (start 32.5188 33.1229) (end 32.5188 33) (width 0.2) (layer "F.Cu") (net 5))
 (segment (start 26.4625 22.5) (end 27.5392 21.4233) (width 0.2) (layer "F.Cu") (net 5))
 (segment (start 38.0441 25.0459) (end 38.0441 21.8766) (width 0.2) (layer "F.Cu") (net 5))
 (segment (start 33.15 27.1142) (end 32.7642 27.1142) (width 0.2) (layer "F.Cu") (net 5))
 (segment (start 32.7 22.5) (end 32.7 22.0483) (width 0.2) (layer "F.Cu") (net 5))
 (segment (start 36.9841 26.1059) (end 38.0441 25.0459) (width 0.2) (layer "F.Cu") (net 5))
 (via (at 32.5188 33.1229) (size 0.6) (drill 0.3) (layers "F.Cu" "B.Cu") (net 5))
 (via (at 32.7642 27.1142) (size 0.6) (drill 0.3) (layers "F.Cu" "B.Cu") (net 5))
 (segment (start 32.5188 27.3596) (end 32.5188 33.1229) (width 0.2) (layer "B.Cu") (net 5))
 (segment (start 32.7642 27.1142) (end 32.5188 27.3596) (width 0.2) (layer "B.Cu") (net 5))
 (segment (start 36.066 37.0012) (end 33.9363 37.0012) (width 0.2) (layer "F.Cu") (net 1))
 (segment (start 23.4231 32.4231) (end 27 36) (width 0.2) (layer "F.Cu") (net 1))
 (segment (start 41.1387 30.4999) (end 41.1387 31.9285) (width 0.2) (layer "F.Cu") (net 1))
 (segment (start 41.1387 31.9285) (end 36.066 37.0012) (width 0.2) (layer "F.Cu") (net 1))
 (segment (start 23.4231 29.9383) (end 23.4231 32.4231) (width 0.2) (layer "F.Cu") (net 1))
 (segment (start 27 38.5) (end 27 37.4844) (width 0.2) (layer "F.Cu") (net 1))
 (segment (start 24.938 29.5001) (end 23.8613 29.5001) (width 0.2) (layer "F.Cu") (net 1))
 (segment (start 27 37.4844) (end 27 36) (width 0.2) (layer "F.Cu") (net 1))
 (segment (start 27 37.4844) (end 31.4219 37.4844) (width 0.2) (layer "F.Cu") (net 1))
 (segment (start 31.4219 37.4844) (end 32.4375 38.5) (width 0.2) (layer "F.Cu") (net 1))
 (segment (start 33.9363 37.0012) (end 32.4375 38.5) (width 0.2) (layer "F.Cu") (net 1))
 (segment (start 23.8613 29.5001) (end 23.4231 29.9383) (width 0.2) (layer "F.Cu") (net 1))
 (segment (start 40.062 30.4999) (end 41.1387 30.4999) (width 0.2) (layer "F.Cu") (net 1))
 (segment (start 24.9375 30.5004) (end 28.9297 30.5004) (width 0.2) (layer "F.Cu") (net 2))
 (segment (start 29 36) (end 26.6122 33.6122) (width 0.2) (layer "F.Cu") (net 2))
 (segment (start 28.9297 30.5004) (end 31.7 27.7301) (width 0.2) (layer "F.Cu") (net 2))
 (segment (start 35 32.4219) (end 35 33.6251) (width 0.2) (layer "F.Cu") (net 2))
 (segment (start 31.7 27.7301) (end 31.7 25.64) (width 0.2) (layer "F.Cu") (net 2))
 (segment (start 35 33.6251) (end 32.6251 36) (width 0.2) (layer "F.Cu") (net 2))
 (segment (start 26.6122 33.6122) (end 25.4992 33.6122) (width 0.2) (layer "F.Cu") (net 2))
 (segment (start 23.8608 31.9738) (end 23.8608 30.5004) (width 0.2) (layer "F.Cu") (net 2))
 (segment (start 25.4992 33.6122) (end 23.8608 31.9738) (width 0.2) (layer "F.Cu") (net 2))
 (segment (start 40.0625 29.4996) (end 37.9223 29.4996) (width 0.2) (layer "F.Cu") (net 2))
 (segment (start 37.9223 29.4996) (end 35 32.4219) (width 0.2) (layer "F.Cu") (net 2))
 (segment (start 24.9375 30.5004) (end 23.8608 30.5004) (width 0.2) (layer "F.Cu") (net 2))
 (segment (start 32.4699 28.5) (end 31.7 27.7301) (width 0.2) (layer "F.Cu") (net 2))
 (segment (start 32.6251 36) (end 29 36) (width 0.2) (layer "F.Cu") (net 2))
 (segment (start 32.5 28.5) (end 32.4699 28.5) (width 0.2) (layer "F.Cu") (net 2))
 (segment (start 31.9513 31.5004) (end 32.3628 31.0889) (width 0.2) (layer "F.Cu") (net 8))
 (segment (start 30.4628 24.0815) (end 30.4628 24.3345) (width 0.2) (layer "F.Cu") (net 8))
 (segment (start 32.3628 31.0889) (end 33.0913 31.8174) (width 0.2) (layer "F.Cu") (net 8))
 (segment (start 31.4 24.82) (end 30.9483 24.82) (width 0.2) (layer "F.Cu") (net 8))
 (segment (start 32.5 30.1) (end 32.5 30.4002) (width 0.2) (layer "F.Cu") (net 8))
 (segment (start 30.2096 38.5) (end 30.313 38.3966) (width 0.2) (layer "F.Cu") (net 8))
 (segment (start 36.8444 28.4996) (end 40.0625 28.4996) (width 0.2) (layer "F.Cu") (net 8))
 (segment (start 32.5 30.4002) (end 32.5 30.9517) (width 0.2) (layer "F.Cu") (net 8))
 (segment (start 32.5 30.4002) (end 30.4654 30.4002) (width 0.2) (layer "F.Cu") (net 8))
 (segment (start 24.9375 31.5004) (end 31.9513 31.5004) (width 0.2) (layer "F.Cu") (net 8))
 (segment (start 32.3628 31.0889) (end 32.5 30.9517) (width 0.2) (layer "F.Cu") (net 8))
 (segment (start 30.4654 30.4002) (end 30.313 30.2478) (width 0.2) (layer "F.Cu") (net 8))
 (segment (start 29 38.5) (end 30.2096 38.5) (width 0.2) (layer "F.Cu") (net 8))
 (segment (start 33.0913 31.8174) (end 33.5266 31.8174) (width 0.2) (layer "F.Cu") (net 8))
 (segment (start 30.4628 24.3345) (end 30.9483 24.82) (width 0.2) (layer "F.Cu") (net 8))
 (segment (start 33.5266 31.8174) (end 36.8444 28.4996) (width 0.2) (layer "F.Cu") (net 8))
 (via (at 30.313 38.3966) (size 0.6) (drill 0.3) (layers "F.Cu" "B.Cu") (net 8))
 (via (at 30.4628 24.0815) (size 0.6) (drill 0.3) (layers "F.Cu" "B.Cu") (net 8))
 (via (at 30.313 30.2478) (size 0.6) (drill 0.3) (layers "F.Cu" "B.Cu") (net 8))
 (segment (start 30.313 30.2478) (end 30.4628 30.098) (width 0.2) (layer "B.Cu") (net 8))
 (segment (start 30.4628 30.098) (end 30.4628 24.0815) (width 0.2) (layer "B.Cu") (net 8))
 (segment (start 30.313 38.3966) (end 30.313 30.2478) (width 0.2) (layer "B.Cu") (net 8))
 (segment (start 37 38.5) (end 34.4375 38.5) (width 0.2) (layer "F.Cu") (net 13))
 (segment (start 37 22.5) (end 33.2 22.5) (width 0.2) (layer "F.Cu") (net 3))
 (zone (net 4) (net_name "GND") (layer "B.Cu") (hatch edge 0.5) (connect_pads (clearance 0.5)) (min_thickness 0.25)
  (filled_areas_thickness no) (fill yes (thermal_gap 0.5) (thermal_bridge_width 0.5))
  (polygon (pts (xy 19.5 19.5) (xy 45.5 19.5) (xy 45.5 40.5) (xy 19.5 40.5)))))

